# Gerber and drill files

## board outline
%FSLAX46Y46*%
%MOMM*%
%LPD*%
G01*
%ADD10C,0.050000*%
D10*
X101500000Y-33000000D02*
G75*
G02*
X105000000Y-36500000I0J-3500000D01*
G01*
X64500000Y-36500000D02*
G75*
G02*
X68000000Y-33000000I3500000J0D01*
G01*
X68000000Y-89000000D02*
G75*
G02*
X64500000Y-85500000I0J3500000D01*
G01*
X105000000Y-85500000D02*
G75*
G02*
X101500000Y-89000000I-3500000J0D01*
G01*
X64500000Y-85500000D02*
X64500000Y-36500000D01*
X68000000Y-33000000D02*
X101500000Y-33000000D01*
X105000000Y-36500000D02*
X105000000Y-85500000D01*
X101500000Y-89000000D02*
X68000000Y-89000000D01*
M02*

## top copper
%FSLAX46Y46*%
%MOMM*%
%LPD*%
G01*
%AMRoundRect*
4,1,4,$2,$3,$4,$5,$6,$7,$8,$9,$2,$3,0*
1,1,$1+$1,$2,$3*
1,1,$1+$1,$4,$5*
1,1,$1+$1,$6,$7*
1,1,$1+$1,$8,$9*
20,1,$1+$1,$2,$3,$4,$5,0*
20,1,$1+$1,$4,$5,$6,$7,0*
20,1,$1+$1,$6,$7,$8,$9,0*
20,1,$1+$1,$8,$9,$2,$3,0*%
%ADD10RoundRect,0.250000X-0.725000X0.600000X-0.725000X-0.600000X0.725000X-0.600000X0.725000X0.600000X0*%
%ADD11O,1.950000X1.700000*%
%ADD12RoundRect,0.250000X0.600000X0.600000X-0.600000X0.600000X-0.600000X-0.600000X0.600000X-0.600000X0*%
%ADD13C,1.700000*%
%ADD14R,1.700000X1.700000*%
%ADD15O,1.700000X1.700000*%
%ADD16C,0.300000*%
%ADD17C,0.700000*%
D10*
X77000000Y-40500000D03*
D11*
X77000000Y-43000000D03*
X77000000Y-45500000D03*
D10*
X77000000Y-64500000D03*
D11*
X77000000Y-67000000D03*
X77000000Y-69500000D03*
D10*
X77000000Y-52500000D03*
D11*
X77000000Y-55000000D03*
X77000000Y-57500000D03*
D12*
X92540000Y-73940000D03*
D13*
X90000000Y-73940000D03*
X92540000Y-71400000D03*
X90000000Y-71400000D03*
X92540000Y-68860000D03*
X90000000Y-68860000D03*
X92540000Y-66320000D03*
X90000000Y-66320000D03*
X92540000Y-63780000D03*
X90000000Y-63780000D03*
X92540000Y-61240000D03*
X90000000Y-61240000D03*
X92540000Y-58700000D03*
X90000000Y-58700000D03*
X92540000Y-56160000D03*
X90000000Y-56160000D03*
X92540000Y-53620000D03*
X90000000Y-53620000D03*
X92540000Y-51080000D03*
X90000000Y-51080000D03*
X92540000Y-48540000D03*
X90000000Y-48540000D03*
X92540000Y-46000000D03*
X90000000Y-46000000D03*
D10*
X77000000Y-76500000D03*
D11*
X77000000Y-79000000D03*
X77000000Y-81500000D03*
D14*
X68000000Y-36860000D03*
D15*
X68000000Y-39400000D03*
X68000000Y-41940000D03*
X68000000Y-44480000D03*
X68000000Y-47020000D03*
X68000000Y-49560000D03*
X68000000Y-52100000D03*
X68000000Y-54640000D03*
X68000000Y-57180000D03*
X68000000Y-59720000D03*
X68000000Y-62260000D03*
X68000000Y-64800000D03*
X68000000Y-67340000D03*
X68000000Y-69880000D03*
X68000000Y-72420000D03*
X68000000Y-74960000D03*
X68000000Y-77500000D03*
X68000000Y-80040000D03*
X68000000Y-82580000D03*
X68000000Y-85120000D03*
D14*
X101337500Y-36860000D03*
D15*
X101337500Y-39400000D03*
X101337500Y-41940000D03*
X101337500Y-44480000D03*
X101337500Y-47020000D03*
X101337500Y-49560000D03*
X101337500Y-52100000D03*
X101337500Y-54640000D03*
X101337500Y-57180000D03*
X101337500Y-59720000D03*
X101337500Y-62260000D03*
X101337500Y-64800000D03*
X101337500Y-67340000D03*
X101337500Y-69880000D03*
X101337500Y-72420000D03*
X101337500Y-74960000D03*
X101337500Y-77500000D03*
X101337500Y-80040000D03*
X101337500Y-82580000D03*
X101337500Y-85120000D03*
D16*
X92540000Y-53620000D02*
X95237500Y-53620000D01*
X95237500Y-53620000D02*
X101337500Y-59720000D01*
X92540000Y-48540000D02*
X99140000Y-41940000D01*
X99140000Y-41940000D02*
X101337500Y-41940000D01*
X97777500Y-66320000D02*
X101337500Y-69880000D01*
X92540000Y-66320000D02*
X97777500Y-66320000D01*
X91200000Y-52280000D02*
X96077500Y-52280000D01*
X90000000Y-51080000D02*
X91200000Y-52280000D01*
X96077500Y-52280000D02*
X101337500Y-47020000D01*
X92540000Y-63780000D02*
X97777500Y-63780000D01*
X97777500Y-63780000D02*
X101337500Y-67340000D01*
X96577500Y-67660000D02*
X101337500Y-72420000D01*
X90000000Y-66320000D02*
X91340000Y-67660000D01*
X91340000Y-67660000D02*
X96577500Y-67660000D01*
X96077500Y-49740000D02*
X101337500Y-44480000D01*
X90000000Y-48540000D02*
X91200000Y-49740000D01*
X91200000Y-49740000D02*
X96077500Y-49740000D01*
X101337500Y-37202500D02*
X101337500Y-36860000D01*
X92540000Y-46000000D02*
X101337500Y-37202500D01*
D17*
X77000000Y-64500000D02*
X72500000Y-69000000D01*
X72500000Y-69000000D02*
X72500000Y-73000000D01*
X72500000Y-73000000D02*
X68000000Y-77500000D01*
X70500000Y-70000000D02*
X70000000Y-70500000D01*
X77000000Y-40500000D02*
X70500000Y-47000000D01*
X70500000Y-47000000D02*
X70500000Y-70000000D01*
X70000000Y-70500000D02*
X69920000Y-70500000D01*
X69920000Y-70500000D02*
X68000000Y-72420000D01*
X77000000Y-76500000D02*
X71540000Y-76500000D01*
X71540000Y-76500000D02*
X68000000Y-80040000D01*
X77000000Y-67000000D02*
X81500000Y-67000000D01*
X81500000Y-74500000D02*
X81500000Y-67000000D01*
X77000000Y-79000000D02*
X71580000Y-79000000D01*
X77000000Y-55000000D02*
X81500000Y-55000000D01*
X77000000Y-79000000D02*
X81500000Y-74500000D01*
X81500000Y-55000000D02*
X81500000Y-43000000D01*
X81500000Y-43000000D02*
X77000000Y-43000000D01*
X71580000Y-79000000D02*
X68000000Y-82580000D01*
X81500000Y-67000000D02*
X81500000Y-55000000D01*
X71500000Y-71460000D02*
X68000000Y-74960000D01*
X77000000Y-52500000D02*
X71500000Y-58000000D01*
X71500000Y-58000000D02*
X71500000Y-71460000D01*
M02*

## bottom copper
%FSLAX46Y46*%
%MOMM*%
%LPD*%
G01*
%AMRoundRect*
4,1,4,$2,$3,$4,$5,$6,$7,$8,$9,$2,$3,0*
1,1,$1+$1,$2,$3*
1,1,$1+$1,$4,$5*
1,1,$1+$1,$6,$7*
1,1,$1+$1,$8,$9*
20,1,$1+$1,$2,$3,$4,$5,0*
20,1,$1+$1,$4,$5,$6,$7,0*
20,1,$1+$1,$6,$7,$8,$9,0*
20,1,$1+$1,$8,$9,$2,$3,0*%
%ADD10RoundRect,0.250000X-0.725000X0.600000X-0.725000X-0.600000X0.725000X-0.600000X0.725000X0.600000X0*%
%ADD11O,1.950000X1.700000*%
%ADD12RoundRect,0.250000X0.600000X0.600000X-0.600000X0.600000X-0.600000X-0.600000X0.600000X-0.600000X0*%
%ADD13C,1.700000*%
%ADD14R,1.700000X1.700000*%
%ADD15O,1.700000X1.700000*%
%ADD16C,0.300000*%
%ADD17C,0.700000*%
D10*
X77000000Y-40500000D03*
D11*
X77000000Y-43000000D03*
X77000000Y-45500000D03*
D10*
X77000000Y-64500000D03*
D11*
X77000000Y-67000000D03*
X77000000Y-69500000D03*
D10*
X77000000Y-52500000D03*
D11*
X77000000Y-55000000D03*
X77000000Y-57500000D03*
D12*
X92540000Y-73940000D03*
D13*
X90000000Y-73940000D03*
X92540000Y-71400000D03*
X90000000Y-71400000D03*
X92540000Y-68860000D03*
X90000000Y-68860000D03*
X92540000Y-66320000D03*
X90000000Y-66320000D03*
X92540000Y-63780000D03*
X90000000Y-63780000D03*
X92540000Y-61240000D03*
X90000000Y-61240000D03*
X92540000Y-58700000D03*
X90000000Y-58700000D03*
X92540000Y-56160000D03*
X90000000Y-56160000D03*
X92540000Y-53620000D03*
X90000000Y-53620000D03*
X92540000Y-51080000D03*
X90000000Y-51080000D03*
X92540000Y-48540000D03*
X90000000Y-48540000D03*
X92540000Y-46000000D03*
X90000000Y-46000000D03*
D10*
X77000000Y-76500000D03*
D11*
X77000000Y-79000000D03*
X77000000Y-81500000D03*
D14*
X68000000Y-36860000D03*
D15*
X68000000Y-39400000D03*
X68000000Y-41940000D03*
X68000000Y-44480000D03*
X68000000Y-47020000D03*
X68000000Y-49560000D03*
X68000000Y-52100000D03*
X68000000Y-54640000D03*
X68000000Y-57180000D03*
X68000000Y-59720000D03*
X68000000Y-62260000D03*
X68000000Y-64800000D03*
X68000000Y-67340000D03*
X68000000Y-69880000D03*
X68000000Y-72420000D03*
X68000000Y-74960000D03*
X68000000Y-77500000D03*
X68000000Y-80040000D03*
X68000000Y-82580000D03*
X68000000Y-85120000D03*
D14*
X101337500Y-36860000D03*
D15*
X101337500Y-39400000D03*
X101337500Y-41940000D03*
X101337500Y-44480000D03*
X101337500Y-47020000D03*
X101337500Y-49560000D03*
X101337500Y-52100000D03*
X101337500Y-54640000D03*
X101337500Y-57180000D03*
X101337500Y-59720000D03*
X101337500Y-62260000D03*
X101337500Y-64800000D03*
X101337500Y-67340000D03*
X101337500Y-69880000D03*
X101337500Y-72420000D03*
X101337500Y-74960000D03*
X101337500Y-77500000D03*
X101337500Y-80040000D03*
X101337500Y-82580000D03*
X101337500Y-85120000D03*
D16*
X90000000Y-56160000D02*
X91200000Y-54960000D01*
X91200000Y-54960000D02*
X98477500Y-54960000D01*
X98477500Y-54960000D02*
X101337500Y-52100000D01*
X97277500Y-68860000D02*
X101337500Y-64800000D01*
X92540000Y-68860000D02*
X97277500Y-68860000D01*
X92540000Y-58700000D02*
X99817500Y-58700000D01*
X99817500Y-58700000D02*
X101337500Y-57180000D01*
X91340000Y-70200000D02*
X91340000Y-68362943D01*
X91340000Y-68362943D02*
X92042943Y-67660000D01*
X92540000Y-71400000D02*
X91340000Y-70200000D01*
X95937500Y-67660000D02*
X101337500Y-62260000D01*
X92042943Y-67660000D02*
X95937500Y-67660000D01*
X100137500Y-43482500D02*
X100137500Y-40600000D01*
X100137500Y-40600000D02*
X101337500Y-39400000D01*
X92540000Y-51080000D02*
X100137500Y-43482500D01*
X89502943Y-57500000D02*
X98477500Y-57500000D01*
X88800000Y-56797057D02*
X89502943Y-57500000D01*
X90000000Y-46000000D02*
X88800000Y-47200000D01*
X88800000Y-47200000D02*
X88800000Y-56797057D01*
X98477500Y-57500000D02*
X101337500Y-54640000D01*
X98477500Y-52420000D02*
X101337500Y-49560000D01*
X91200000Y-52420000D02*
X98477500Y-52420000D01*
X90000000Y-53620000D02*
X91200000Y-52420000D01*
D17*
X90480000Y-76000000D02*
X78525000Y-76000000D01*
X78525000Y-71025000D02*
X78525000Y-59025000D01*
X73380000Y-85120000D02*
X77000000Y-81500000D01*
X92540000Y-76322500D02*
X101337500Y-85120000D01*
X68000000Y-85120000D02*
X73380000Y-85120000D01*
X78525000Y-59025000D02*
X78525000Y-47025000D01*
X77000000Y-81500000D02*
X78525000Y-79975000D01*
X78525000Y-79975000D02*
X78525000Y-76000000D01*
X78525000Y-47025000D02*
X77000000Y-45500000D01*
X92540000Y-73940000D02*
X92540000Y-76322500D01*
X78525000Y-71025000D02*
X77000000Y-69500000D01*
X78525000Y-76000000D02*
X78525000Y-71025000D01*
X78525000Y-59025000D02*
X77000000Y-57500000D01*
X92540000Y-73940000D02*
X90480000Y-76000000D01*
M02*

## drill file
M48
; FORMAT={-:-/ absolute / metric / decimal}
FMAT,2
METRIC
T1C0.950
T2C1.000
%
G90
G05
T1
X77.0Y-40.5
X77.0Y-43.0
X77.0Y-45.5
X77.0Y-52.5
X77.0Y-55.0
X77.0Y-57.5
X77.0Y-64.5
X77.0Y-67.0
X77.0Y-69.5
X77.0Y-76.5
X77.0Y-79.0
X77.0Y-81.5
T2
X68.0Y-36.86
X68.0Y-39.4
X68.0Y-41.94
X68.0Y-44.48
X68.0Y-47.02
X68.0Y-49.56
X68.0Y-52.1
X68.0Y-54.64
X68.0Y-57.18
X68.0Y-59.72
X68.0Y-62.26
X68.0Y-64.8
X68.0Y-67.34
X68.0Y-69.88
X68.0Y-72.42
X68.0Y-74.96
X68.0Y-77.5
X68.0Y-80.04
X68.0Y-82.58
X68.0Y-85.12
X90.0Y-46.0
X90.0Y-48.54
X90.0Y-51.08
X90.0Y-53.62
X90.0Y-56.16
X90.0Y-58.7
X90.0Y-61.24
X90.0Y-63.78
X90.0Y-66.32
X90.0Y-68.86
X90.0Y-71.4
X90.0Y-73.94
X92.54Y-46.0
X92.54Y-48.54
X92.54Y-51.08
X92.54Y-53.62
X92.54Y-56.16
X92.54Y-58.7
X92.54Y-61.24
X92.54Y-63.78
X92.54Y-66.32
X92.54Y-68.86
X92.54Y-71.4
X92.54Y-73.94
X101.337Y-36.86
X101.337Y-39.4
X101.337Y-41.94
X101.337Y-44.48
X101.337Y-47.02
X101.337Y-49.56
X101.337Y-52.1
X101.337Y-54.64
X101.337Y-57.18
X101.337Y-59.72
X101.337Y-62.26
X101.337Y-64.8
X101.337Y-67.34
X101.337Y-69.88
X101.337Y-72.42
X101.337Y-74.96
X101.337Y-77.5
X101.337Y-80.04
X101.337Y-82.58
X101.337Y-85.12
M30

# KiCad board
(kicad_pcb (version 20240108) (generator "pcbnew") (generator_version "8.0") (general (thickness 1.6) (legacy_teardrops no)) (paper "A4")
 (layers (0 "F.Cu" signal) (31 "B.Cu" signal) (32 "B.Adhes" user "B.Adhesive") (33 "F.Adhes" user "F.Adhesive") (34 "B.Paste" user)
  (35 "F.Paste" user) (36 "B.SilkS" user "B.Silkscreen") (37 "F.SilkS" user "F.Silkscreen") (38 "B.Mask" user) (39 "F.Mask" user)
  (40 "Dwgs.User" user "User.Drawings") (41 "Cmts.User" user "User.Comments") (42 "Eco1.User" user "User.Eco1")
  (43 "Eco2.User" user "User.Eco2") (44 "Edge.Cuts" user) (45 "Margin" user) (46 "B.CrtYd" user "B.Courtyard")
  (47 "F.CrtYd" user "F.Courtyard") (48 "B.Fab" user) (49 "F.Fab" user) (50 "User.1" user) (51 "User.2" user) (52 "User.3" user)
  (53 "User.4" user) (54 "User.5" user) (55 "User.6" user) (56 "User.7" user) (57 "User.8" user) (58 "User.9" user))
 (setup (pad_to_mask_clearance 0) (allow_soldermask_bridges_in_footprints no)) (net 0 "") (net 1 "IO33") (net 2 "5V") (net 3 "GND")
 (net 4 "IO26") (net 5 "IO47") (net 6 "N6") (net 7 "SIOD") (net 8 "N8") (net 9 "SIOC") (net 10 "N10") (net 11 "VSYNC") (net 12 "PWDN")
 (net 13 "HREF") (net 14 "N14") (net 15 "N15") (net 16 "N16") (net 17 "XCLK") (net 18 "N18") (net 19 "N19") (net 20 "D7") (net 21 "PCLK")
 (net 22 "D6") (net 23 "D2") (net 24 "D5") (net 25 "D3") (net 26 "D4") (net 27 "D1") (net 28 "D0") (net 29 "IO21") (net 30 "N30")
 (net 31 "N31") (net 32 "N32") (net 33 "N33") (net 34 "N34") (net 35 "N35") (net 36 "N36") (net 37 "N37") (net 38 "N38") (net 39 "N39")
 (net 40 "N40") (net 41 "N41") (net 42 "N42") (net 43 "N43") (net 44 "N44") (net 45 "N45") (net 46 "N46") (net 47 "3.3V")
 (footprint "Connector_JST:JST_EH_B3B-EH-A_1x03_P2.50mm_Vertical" (layer "F.Cu") (at 77 40.5 -90)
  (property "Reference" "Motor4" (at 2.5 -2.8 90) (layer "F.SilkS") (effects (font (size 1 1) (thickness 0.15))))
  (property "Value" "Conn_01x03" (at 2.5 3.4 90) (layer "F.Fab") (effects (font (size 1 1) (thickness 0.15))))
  (pad "1" thru_hole roundrect (at 0 0 270) (size 1.7 1.95) (drill 0.95) (layers "*.Cu" "*.Mask") (remove_unused_layers no)
   (roundrect_rratio 0.147059) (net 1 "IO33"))
  (pad "2" thru_hole oval (at 2.5 0 270) (size 1.7 1.95) (drill 0.95) (layers "*.Cu" "*.Mask") (remove_unused_layers no) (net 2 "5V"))
  (pad "3" thru_hole oval (at 5 0 270) (size 1.7 1.95) (drill 0.95) (layers "*.Cu" "*.Mask") (remove_unused_layers no) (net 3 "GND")))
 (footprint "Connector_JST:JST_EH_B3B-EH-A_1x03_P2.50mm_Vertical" (layer "F.Cu") (at 77 64.5 -90)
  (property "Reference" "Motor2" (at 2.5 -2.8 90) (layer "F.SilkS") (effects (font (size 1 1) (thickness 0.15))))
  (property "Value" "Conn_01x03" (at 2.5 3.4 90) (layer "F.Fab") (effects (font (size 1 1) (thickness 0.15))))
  (pad "1" thru_hole roundrect (at 0 0 270) (size 1.7 1.95) (drill 0.95) (layers "*.Cu" "*.Mask") (remove_unused_layers no)
   (roundrect_rratio 0.147059) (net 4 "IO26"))
  (pad "2" thru_hole oval (at 2.5 0 270) (size 1.7 1.95) (drill 0.95) (layers "*.Cu" "*.Mask") (remove_unused_layers no) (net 2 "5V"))
  (pad "3" thru_hole oval (at 5 0 270) (size 1.7 1.95) (drill 0.95) (layers "*.Cu" "*.Mask") (remove_unused_layers no) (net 3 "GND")))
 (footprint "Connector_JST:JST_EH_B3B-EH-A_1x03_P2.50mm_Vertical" (layer "F.Cu") (at 77 52.5 -90)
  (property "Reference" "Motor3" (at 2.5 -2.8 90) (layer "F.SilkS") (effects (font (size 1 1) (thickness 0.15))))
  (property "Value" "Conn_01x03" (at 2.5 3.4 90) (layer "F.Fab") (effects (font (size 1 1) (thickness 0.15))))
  (pad "1" thru_hole roundrect (at 0 0 270) (size 1.7 1.95) (drill 0.95) (layers "*.Cu" "*.Mask") (remove_unused_layers no)
   (roundrect_rratio 0.147059) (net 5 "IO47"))
  (pad "2" thru_hole oval (at 2.5 0 270) (size 1.7 1.95) (drill 0.95) (layers "*.Cu" "*.Mask") (remove_unused_layers no) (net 2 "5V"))
  (pad "3" thru_hole oval (at 5 0 270) (size 1.7 1.95) (drill 0.95) (layers "*.Cu" "*.Mask") (remove_unused_layers no) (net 3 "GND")))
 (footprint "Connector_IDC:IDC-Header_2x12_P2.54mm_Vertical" (layer "F.Cu") (at 92.54 73.94 180)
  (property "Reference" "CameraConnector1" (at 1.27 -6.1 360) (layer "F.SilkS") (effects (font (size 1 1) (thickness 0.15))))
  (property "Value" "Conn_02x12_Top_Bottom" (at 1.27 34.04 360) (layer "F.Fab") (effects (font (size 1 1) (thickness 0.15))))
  (pad "1" thru_hole roundrect (at 0 0 180) (size 1.7 1.7) (drill 1) (layers "*.Cu" "*.Mask") (remove_unused_layers no)
   (roundrect_rratio 0.147059) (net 3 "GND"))
  (pad "2" thru_hole circle (at 2.54 0 180) (size 1.7 1.7) (drill 1) (layers "*.Cu" "*.Mask") (remove_unused_layers no) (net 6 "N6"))
  (pad "3" thru_hole circle (at 0 2.54 180) (size 1.7 1.7) (drill 1) (layers "*.Cu" "*.Mask") (remove_unused_layers no) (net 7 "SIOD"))
  (pad "4" thru_hole circle (at 2.54 2.54 180) (size 1.7 1.7) (drill 1) (layers "*.Cu" "*.Mask") (remove_unused_layers no) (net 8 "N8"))
  (pad "5" thru_hole circle (at 0 5.08 180) (size 1.7 1.7) (drill 1) (layers "*.Cu" "*.Mask") (remove_unused_layers no) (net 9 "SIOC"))
  (pad "6" thru_hole circle (at 2.54 5.08 180) (size 1.7 1.7) (drill 1) (layers "*.Cu" "*.Mask") (remove_unused_layers no) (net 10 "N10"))
  (pad "7" thru_hole circle (at 0 7.62 180) (size 1.7 1.7) (drill 1) (layers "*.Cu" "*.Mask") (remove_unused_layers no) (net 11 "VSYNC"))
  (pad "8" thru_hole circle (at 2.54 7.62 180) (size 1.7 1.7) (drill 1) (layers "*.Cu" "*.Mask") (remove_unused_layers no) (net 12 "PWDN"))
  (pad "9" thru_hole circle (at 0 10.16 180) (size 1.7 1.7) (drill 1) (layers "*.Cu" "*.Mask") (remove_unused_layers no) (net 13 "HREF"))
  (pad "10" thru_hole circle (at 2.54 10.16 180) (size 1.7 1.7) (drill 1) (layers "*.Cu" "*.Mask") (remove_unused_layers no) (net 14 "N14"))
  (pad "11" thru_hole circle (at 0 12.7 180) (size 1.7 1.7) (drill 1) (layers "*.Cu" "*.Mask") (remove_unused_layers no) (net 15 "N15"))
  (pad "12" thru_hole circle (at 2.54 12.7 180) (size 1.7 1.7) (drill 1) (layers "*.Cu" "*.Mask") (remove_unused_layers no) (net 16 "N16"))
  (pad "13" thru_hole circle (at 0 15.24 180) (size 1.7 1.7) (drill 1) (layers "*.Cu" "*.Mask") (remove_unused_layers no) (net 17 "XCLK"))
  (pad "14" thru_hole circle (at 2.54 15.24 180) (size 1.7 1.7) (drill 1) (layers "*.Cu" "*.Mask") (remove_unused_layers no) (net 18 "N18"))
  (pad "15" thru_hole circle (at 0 17.78 180) (size 1.7 1.7) (drill 1) (layers "*.Cu" "*.Mask") (remove_unused_layers no) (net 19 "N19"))
  (pad "16" thru_hole circle (at 2.54 17.78 180) (size 1.7 1.7) (drill 1) (layers "*.Cu" "*.Mask") (remove_unused_layers no) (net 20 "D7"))
  (pad "17" thru_hole circle (at 0 20.32 180) (size 1.7 1.7) (drill 1) (layers "*.Cu" "*.Mask") (remove_unused_layers no) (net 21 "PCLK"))
  (pad "18" thru_hole circle (at 2.54 20.32 180) (size 1.7 1.7) (drill 1) (layers "*.Cu" "*.Mask") (remove_unused_layers no) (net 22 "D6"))
  (pad "19" thru_hole circle (at 0 22.86 180) (size 1.7 1.7) (drill 1) (layers "*.Cu" "*.Mask") (remove_unused_layers no) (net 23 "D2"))
  (pad "20" thru_hole circle (at 2.54 22.86 180) (size 1.7 1.7) (drill 1) (layers "*.Cu" "*.Mask") (remove_unused_layers no) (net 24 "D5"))
  (pad "21" thru_hole circle (at 0 25.4 180) (size 1.7 1.7) (drill 1) (layers "*.Cu" "*.Mask") (remove_unused_layers no) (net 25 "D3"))
  (pad "22" thru_hole circle (at 2.54 25.4 180) (size 1.7 1.7) (drill 1) (layers "*.Cu" "*.Mask") (remove_unused_layers no) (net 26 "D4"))
  (pad "23" thru_hole circle (at 0 27.94 180) (size 1.7 1.7) (drill 1) (layers "*.Cu" "*.Mask") (remove_unused_layers no) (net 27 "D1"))
  (pad "24" thru_hole circle (at 2.54 27.94 180) (size 1.7 1.7) (drill 1) (layers "*.Cu" "*.Mask") (remove_unused_layers no) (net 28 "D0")))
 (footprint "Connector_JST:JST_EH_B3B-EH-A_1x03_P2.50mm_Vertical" (layer "F.Cu") (at 77 76.5 -90)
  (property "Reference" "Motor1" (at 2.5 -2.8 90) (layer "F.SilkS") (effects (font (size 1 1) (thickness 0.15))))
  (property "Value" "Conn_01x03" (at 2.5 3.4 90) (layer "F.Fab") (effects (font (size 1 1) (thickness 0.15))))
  (pad "1" thru_hole roundrect (at 0 0 270) (size 1.7 1.95) (drill 0.95) (layers "*.Cu" "*.Mask") (remove_unused_layers no)
   (roundrect_rratio 0.147059) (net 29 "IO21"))
  (pad "2" thru_hole oval (at 2.5 0 270) (size 1.7 1.95) (drill 0.95) (layers "*.Cu" "*.Mask") (remove_unused_layers no) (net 2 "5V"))
  (pad "3" thru_hole oval (at 5 0 270) (size 1.7 1.95) (drill 0.95) (layers "*.Cu" "*.Mask") (remove_unused_layers no) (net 3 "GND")))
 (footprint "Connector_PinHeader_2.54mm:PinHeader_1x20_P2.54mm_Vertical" (layer "B.Cu") (at 68 36.86 180)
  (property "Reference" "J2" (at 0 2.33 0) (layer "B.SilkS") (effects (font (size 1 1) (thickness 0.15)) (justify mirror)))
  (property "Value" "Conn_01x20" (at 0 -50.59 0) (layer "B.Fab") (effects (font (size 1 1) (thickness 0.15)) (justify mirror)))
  (pad "1" thru_hole rect (at 0 0 180) (size 1.7 1.7) (drill 1) (layers "*.Cu" "*.Mask") (remove_unused_layers no) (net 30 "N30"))
  (pad "2" thru_hole oval (at 0 -2.54 180) (size 1.7 1.7) (drill 1) (layers "*.Cu" "*.Mask") (remove_unused_layers no) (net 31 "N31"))
  (pad "3" thru_hole oval (at 0 -5.08 180) (size 1.7 1.7) (drill 1) (layers "*.Cu" "*.Mask") (remove_unused_layers no) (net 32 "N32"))
  (pad "4" thru_hole oval (at 0 -7.62 180) (size 1.7 1.7) (drill 1) (layers "*.Cu" "*.Mask") (remove_unused_layers no) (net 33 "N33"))
  (pad "5" thru_hole oval (at 0 -10.16 180) (size 1.7 1.7) (drill 1) (layers "*.Cu" "*.Mask") (remove_unused_layers no) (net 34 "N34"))
  (pad "6" thru_hole oval (at 0 -12.7 180) (size 1.7 1.7) (drill 1) (layers "*.Cu" "*.Mask") (remove_unused_layers no) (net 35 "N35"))
  (pad "7" thru_hole oval (at 0 -15.24 180) (size 1.7 1.7) (drill 1) (layers "*.Cu" "*.Mask") (remove_unused_layers no) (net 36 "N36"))
  (pad "8" thru_hole oval (at 0 -17.78 180) (size 1.7 1.7) (drill 1) (layers "*.Cu" "*.Mask") (remove_unused_layers no) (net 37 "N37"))
  (pad "9" thru_hole oval (at 0 -20.32 180) (size 1.7 1.7) (drill 1) (layers "*.Cu" "*.Mask") (remove_unused_layers no) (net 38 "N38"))
  (pad "10" thru_hole oval (at 0 -22.86 180) (size 1.7 1.7) (drill 1) (layers "*.Cu" "*.Mask") (remove_unused_layers no) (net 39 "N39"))
  (pad "11" thru_hole oval (at 0 -25.4 180) (size 1.7 1.7) (drill 1) (layers "*.Cu" "*.Mask") (remove_unused_layers no) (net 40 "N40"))
  (pad "12" thru_hole oval (at 0 -27.94 180) (size 1.7 1.7) (drill 1) (layers "*.Cu" "*.Mask") (remove_unused_layers no) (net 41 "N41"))
  (pad "13" thru_hole oval (at 0 -30.48 180) (size 1.7 1.7) (drill 1) (layers "*.Cu" "*.Mask") (remove_unused_layers no) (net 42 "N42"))
  (pad "14" thru_hole oval (at 0 -33.02 180) (size 1.7 1.7) (drill 1) (layers "*.Cu" "*.Mask") (remove_unused_layers no) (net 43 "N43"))
  (pad "15" thru_hole oval (at 0 -35.56 180) (size 1.7 1.7) (drill 1) (layers "*.Cu" "*.Mask") (remove_unused_layers no) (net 1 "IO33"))
  (pad "16" thru_hole oval (at 0 -38.1 180) (size 1.7 1.7) (drill 1) (layers "*.Cu" "*.Mask") (remove_unused_layers no) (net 5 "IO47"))
  (pad "17" thru_hole oval (at 0 -40.64 180) (size 1.7 1.7) (drill 1) (layers "*.Cu" "*.Mask") (remove_unused_layers no) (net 4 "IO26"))
  (pad "18" thru_hole oval (at 0 -43.18 180) (size 1.7 1.7) (drill 1) (layers "*.Cu" "*.Mask") (remove_unused_layers no) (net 29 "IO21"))
  (pad "19" thru_hole oval (at 0 -45.72 180) (size 1.7 1.7) (drill 1) (layers "*.Cu" "*.Mask") (remove_unused_layers no) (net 2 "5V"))
  (pad "20" thru_hole oval (at 0 -48.26 180) (size 1.7 1.7) (drill 1) (layers "*.Cu" "*.Mask") (remove_unused_layers no) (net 3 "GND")))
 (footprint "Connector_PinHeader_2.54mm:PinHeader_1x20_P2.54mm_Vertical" (layer "B.Cu") (at 101.3375 36.86 180)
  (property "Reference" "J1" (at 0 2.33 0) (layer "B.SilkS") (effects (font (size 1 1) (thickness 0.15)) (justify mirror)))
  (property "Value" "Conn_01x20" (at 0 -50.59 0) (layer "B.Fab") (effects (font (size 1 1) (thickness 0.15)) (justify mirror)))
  (pad "1" thru_hole rect (at 0 0 180) (size 1.7 1.7) (drill 1) (layers "*.Cu" "*.Mask") (remove_unused_layers no) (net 27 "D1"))
  (pad "2" thru_hole oval (at 0 -2.54 180) (size 1.7 1.7) (drill 1) (layers "*.Cu" "*.Mask") (remove_unused_layers no) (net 23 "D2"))
  (pad "3" thru_hole oval (at 0 -5.08 180) (size 1.7 1.7) (drill 1) (layers "*.Cu" "*.Mask") (remove_unused_layers no) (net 25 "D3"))
  (pad "4" thru_hole oval (at 0 -7.62 180) (size 1.7 1.7) (drill 1) (layers "*.Cu" "*.Mask") (remove_unused_layers no) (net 26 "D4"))
  (pad "5" thru_hole oval (at 0 -10.16 180) (size 1.7 1.7) (drill 1) (layers "*.Cu" "*.Mask") (remove_unused_layers no) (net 24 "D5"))
  (pad "6" thru_hole oval (at 0 -12.7 180) (size 1.7 1.7) (drill 1) (layers "*.Cu" "*.Mask") (remove_unused_layers no) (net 22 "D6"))
  (pad "7" thru_hole oval (at 0 -15.24 180) (size 1.7 1.7) (drill 1) (layers "*.Cu" "*.Mask") (remove_unused_layers no) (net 20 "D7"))
  (pad "8" thru_hole oval (at 0 -17.78 180) (size 1.7 1.7) (drill 1) (layers "*.Cu" "*.Mask") (remove_unused_layers no) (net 28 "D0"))
  (pad "9" thru_hole oval (at 0 -20.32 180) (size 1.7 1.7) (drill 1) (layers "*.Cu" "*.Mask") (remove_unused_layers no) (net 17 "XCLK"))
  (pad "10" thru_hole oval (at 0 -22.86 180) (size 1.7 1.7) (drill 1) (layers "*.Cu" "*.Mask") (remove_unused_layers no) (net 21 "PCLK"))
  (pad "11" thru_hole oval (at 0 -25.4 180) (size 1.7 1.7) (drill 1) (layers "*.Cu" "*.Mask") (remove_unused_layers no) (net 7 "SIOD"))
  (pad "12" thru_hole oval (at 0 -27.94 180) (size 1.7 1.7) (drill 1) (layers "*.Cu" "*.Mask") (remove_unused_layers no) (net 9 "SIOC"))
  (pad "13" thru_hole oval (at 0 -30.48 180) (size 1.7 1.7) (drill 1) (layers "*.Cu" "*.Mask") (remove_unused_layers no) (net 13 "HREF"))
  (pad "14" thru_hole oval (at 0 -33.02 180) (size 1.7 1.7) (drill 1) (layers "*.Cu" "*.Mask") (remove_unused_layers no) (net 11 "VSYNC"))
  (pad "15" thru_hole oval (at 0 -35.56 180) (size 1.7 1.7) (drill 1) (layers "*.Cu" "*.Mask") (remove_unused_layers no) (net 12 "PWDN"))
  (pad "16" thru_hole oval (at 0 -38.1 180) (size 1.7 1.7) (drill 1) (layers "*.Cu" "*.Mask") (remove_unused_layers no) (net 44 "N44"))
  (pad "17" thru_hole oval (at 0 -40.64 180) (size 1.7 1.7) (drill 1) (layers "*.Cu" "*.Mask") (remove_unused_layers no) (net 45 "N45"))
  (pad "18" thru_hole oval (at 0 -43.18 180) (size 1.7 1.7) (drill 1) (layers "*.Cu" "*.Mask") (remove_unused_layers no) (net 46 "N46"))
  (pad "19" thru_hole oval (at 0 -45.72 180) (size 1.7 1.7) (drill 1) (layers "*.Cu" "*.Mask") (remove_unused_layers no) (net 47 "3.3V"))
  (pad "20" thru_hole oval (at 0 -48.26 180) (size 1.7 1.7) (drill 1) (layers "*.Cu" "*.Mask") (remove_unused_layers no) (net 3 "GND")))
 (gr_arc (start 101.5 33) (mid 103.974874 34.025126) (end 105 36.5) (stroke (width 0.05) (type default)) (layer "Edge.Cuts"))
 (gr_arc (start 64.5 36.5) (mid 65.525126 34.025126) (end 68 33) (stroke (width 0.05) (type default)) (layer "Edge.Cuts"))
 (gr_arc (start 68 89) (mid 65.525126 87.974874) (end 64.5 85.5) (stroke (width 0.05) (type default)) (layer "Edge.Cuts"))
 (gr_arc (start 105 85.5) (mid 103.974874 87.974874) (end 101.5 89) (stroke (width 0.05) (type default)) (layer "Edge.Cuts"))
 (gr_line (start 64.5 85.5) (end 64.5 36.5) (stroke (width 0.05) (type default)) (layer "Edge.Cuts"))
 (gr_line (start 68 33) (end 101.5 33) (stroke (width 0.05) (type default)) (layer "Edge.Cuts"))
 (gr_line (start 105 36.5) (end 105 85.5) (stroke (width 0.05) (type default)) (layer "Edge.Cuts"))
 (gr_line (start 101.5 89) (end 68 89) (stroke (width 0.05) (type default)) (layer "Edge.Cuts"))
 (segment (start 90 56.16) (end 91.2 54.96) (width 0.3) (layer "B.Cu") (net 20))
 (segment (start 91.2 54.96) (end 98.4775 54.96) (width 0.3) (layer "B.Cu") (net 20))
 (segment (start 98.4775 54.96) (end 101.3375 52.1) (width 0.3) (layer "B.Cu") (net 20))
 (segment (start 92.54 53.62) (end 95.2375 53.62) (width 0.3) (layer "F.Cu") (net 21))
 (segment (start 95.2375 53.62) (end 101.3375 59.72) (width 0.3) (layer "F.Cu") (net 21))
 (segment (start 92.54 48.54) (end 99.14 41.94) (width 0.3) (layer "F.Cu") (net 25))
 (segment (start 99.14 41.94) (end 101.3375 41.94) (width 0.3) (layer "F.Cu") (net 25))
 (segment (start 97.7775 66.32) (end 101.3375 69.88) (width 0.3) (layer "F.Cu") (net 11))
 (segment (start 92.54 66.32) (end 97.7775 66.32) (width 0.3) (layer "F.Cu") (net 11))
 (segment (start 97.2775 68.86) (end 101.3375 64.8) (width 0.3) (layer "B.Cu") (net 9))
 (segment (start 92.54 68.86) (end 97.2775 68.86) (width 0.3) (layer "B.Cu") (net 9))
 (segment (start 91.2 52.28) (end 96.0775 52.28) (width 0.3) (layer "F.Cu") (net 24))
 (segment (start 90 51.08) (end 91.2 52.28) (width 0.3) (layer "F.Cu") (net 24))
 (segment (start 96.0775 52.28) (end 101.3375 47.02) (width 0.3) (layer "F.Cu") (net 24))
 (segment (start 92.54 58.7) (end 99.8175 58.7) (width 0.3) (layer "B.Cu") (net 17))
 (segment (start 99.8175 58.7) (end 101.3375 57.18) (width 0.3) (layer "B.Cu") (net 17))
 (segment (start 92.54 63.78) (end 97.7775 63.78) (width 0.3) (layer "F.Cu") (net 13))
 (segment (start 97.7775 63.78) (end 101.3375 67.34) (width 0.3) (layer "F.Cu") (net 13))
 (segment (start 96.5775 67.66) (end 101.3375 72.42) (width 0.3) (layer "F.Cu") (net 12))
 (segment (start 90 66.32) (end 91.34 67.66) (width 0.3) (layer "F.Cu") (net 12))
 (segment (start 91.34 67.66) (end 96.5775 67.66) (width 0.3) (layer "F.Cu") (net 12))
 (segment (start 96.0775 49.74) (end 101.3375 44.48) (width 0.3) (layer "F.Cu") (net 26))
 (segment (start 90 48.54) (end 91.2 49.74) (width 0.3) (layer "F.Cu") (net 26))
 (segment (start 91.2 49.74) (end 96.0775 49.74) (width 0.3) (layer "F.Cu") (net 26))
 (segment (start 91.34 70.2) (end 91.34 68.362943) (width 0.3) (layer "B.Cu") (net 7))
 (segment (start 91.34 68.362943) (end 92.042943 67.66) (width 0.3) (layer "B.Cu") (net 7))
 (segment (start 92.54 71.4) (end 91.34 70.2) (width 0.3) (layer "B.Cu") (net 7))
 (segment (start 95.9375 67.66) (end 101.3375 62.26) (width 0.3) (layer "B.Cu") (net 7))
 (segment (start 92.042943 67.66) (end 95.9375 67.66) (width 0.3) (layer "B.Cu") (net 7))
 (segment (start 100.1375 43.4825) (end 100.1375 40.6) (width 0.3) (layer "B.Cu") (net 23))
 (segment (start 100.1375 40.6) (end 101.3375 39.4) (width 0.3) (layer "B.Cu") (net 23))
 (segment (start 92.54 51.08) (end 100.1375 43.4825) (width 0.3) (layer "B.Cu") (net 23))
 (segment (start 101.3375 37.2025) (end 101.3375 36.86) (width 0.3) (layer "F.Cu") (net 27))
 (segment (start 92.54 46) (end 101.3375 37.2025) (width 0.3) (layer "F.Cu") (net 27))
 (segment (start 89.502943 57.5) (end 98.4775 57.5) (width 0.3) (layer "B.Cu") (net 28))
 (segment (start 88.8 56.797057) (end 89.502943 57.5) (width 0.3) (layer "B.Cu") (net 28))
 (segment (start 90 46) (end 88.8 47.2) (width 0.3) (layer "B.Cu") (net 28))
 (segment (start 88.8 47.2) (end 88.8 56.797057) (width 0.3) (layer "B.Cu") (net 28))
 (segment (start 98.4775 57.5) (end 101.3375 54.64) (width 0.3) (layer "B.Cu") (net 28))
 (segment (start 98.4775 52.42) (end 101.3375 49.56) (width 0.3) (layer "B.Cu") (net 22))
 (segment (start 91.2 52.42) (end 98.4775 52.42) (width 0.3) (layer "B.Cu") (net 22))
 (segment (start 90 53.62) (end 91.2 52.42) (width 0.3) (layer "B.Cu") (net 22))
 (segment (start 90.48 76) (end 78.525 76) (width 0.7) (layer "B.Cu") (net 3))
 (segment (start 78.525 71.025) (end 78.525 59.025) (width 0.7) (layer "B.Cu") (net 3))
 (segment (start 73.38 85.12) (end 77 81.5) (width 0.7) (layer "B.Cu") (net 3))
 (segment (start 92.54 76.3225) (end 101.3375 85.12) (width 0.7) (layer "B.Cu") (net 3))
 (segment (start 68 85.12) (end 73.38 85.12) (width 0.7) (layer "B.Cu") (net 3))
 (segment (start 78.525 59.025) (end 78.525 47.025) (width 0.7) (layer "B.Cu") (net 3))
 (segment (start 77 81.5) (end 78.525 79.975) (width 0.7) (layer "B.Cu") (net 3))
 (segment (start 78.525 79.975) (end 78.525 76) (width 0.7) (layer "B.Cu") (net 3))
 (segment (start 78.525 47.025) (end 77 45.5) (width 0.7) (layer "B.Cu") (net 3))
 (segment (start 92.54 73.94) (end 92.54 76.3225) (width 0.7) (layer "B.Cu") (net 3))
 (segment (start 78.525 71.025) (end 77 69.5) (width 0.7) (layer "B.Cu") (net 3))
 (segment (start 78.525 76) (end 78.525 71.025) (width 0.7) (layer "B.Cu") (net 3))
 (segment (start 78.525 59.025) (end 77 57.5) (width 0.7) (layer "B.Cu") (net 3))
 (segment (start 92.54 73.94) (end 90.48 76) (width 0.7) (layer "B.Cu") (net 3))
 (segment (start 77 64.5) (end 72.5 69) (width 0.7) (layer "F.Cu") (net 4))
 (segment (start 72.5 69) (end 72.5 73) (width 0.7) (layer "F.Cu") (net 4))
 (segment (start 72.5 73) (end 68 77.5) (width 0.7) (layer "F.Cu") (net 4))
 (segment (start 70.5 70) (end 70 70.5) (width 0.7) (layer "F.Cu") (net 1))
 (segment (start 77 40.5) (end 70.5 47) (width 0.7) (layer "F.Cu") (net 1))
 (segment (start 70.5 47) (end 70.5 70) (width 0.7) (layer "F.Cu") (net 1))
 (segment (start 70 70.5) (end 69.92 70.5) (width 0.7) (layer "F.Cu") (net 1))
 (segment (start 69.92 70.5) (end 68 72.42) (width 0.7) (layer "F.Cu") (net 1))
 (segment (start 77 76.5) (end 71.54 76.5) (width 0.7) (layer "F.Cu") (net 29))
 (segment (start 71.54 76.5) (end 68 80.04) (width 0.7) (layer "F.Cu") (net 29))
 (segment (start 77 67) (end 81.5 67) (width 0.7) (layer "F.Cu") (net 2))
 (segment (start 81.5 74.5) (end 81.5 67) (width 0.7) (layer "F.Cu") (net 2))
 (segment (start 77 79) (end 71.58 79) (width 0.7) (layer "F.Cu") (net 2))
 (segment (start 77 55) (end 81.5 55) (width 0.7) (layer "F.Cu") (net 2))
 (segment (start 77 79) (end 81.5 74.5) (width 0.7) (layer "F.Cu") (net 2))
 (segment (start 81.5 55) (end 81.5 43) (width 0.7) (layer "F.Cu") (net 2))
 (segment (start 81.5 43) (end 77 43) (width 0.7) (layer "F.Cu") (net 2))
 (segment (start 71.58 79) (end 68 82.58) (width 0.7) (layer "F.Cu") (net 2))
 (segment (start 81.5 67) (end 81.5 55) (width 0.7) (layer "F.Cu") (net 2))
 (segment (start 71.5 71.46) (end 68 74.96) (width 0.7) (layer "F.Cu") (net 5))
 (segment (start 77 52.5) (end 71.5 58) (width 0.7) (layer "F.Cu") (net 5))
 (segment (start 71.5 58) (end 71.5 71.46) (width 0.7) (layer "F.Cu") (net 5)))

